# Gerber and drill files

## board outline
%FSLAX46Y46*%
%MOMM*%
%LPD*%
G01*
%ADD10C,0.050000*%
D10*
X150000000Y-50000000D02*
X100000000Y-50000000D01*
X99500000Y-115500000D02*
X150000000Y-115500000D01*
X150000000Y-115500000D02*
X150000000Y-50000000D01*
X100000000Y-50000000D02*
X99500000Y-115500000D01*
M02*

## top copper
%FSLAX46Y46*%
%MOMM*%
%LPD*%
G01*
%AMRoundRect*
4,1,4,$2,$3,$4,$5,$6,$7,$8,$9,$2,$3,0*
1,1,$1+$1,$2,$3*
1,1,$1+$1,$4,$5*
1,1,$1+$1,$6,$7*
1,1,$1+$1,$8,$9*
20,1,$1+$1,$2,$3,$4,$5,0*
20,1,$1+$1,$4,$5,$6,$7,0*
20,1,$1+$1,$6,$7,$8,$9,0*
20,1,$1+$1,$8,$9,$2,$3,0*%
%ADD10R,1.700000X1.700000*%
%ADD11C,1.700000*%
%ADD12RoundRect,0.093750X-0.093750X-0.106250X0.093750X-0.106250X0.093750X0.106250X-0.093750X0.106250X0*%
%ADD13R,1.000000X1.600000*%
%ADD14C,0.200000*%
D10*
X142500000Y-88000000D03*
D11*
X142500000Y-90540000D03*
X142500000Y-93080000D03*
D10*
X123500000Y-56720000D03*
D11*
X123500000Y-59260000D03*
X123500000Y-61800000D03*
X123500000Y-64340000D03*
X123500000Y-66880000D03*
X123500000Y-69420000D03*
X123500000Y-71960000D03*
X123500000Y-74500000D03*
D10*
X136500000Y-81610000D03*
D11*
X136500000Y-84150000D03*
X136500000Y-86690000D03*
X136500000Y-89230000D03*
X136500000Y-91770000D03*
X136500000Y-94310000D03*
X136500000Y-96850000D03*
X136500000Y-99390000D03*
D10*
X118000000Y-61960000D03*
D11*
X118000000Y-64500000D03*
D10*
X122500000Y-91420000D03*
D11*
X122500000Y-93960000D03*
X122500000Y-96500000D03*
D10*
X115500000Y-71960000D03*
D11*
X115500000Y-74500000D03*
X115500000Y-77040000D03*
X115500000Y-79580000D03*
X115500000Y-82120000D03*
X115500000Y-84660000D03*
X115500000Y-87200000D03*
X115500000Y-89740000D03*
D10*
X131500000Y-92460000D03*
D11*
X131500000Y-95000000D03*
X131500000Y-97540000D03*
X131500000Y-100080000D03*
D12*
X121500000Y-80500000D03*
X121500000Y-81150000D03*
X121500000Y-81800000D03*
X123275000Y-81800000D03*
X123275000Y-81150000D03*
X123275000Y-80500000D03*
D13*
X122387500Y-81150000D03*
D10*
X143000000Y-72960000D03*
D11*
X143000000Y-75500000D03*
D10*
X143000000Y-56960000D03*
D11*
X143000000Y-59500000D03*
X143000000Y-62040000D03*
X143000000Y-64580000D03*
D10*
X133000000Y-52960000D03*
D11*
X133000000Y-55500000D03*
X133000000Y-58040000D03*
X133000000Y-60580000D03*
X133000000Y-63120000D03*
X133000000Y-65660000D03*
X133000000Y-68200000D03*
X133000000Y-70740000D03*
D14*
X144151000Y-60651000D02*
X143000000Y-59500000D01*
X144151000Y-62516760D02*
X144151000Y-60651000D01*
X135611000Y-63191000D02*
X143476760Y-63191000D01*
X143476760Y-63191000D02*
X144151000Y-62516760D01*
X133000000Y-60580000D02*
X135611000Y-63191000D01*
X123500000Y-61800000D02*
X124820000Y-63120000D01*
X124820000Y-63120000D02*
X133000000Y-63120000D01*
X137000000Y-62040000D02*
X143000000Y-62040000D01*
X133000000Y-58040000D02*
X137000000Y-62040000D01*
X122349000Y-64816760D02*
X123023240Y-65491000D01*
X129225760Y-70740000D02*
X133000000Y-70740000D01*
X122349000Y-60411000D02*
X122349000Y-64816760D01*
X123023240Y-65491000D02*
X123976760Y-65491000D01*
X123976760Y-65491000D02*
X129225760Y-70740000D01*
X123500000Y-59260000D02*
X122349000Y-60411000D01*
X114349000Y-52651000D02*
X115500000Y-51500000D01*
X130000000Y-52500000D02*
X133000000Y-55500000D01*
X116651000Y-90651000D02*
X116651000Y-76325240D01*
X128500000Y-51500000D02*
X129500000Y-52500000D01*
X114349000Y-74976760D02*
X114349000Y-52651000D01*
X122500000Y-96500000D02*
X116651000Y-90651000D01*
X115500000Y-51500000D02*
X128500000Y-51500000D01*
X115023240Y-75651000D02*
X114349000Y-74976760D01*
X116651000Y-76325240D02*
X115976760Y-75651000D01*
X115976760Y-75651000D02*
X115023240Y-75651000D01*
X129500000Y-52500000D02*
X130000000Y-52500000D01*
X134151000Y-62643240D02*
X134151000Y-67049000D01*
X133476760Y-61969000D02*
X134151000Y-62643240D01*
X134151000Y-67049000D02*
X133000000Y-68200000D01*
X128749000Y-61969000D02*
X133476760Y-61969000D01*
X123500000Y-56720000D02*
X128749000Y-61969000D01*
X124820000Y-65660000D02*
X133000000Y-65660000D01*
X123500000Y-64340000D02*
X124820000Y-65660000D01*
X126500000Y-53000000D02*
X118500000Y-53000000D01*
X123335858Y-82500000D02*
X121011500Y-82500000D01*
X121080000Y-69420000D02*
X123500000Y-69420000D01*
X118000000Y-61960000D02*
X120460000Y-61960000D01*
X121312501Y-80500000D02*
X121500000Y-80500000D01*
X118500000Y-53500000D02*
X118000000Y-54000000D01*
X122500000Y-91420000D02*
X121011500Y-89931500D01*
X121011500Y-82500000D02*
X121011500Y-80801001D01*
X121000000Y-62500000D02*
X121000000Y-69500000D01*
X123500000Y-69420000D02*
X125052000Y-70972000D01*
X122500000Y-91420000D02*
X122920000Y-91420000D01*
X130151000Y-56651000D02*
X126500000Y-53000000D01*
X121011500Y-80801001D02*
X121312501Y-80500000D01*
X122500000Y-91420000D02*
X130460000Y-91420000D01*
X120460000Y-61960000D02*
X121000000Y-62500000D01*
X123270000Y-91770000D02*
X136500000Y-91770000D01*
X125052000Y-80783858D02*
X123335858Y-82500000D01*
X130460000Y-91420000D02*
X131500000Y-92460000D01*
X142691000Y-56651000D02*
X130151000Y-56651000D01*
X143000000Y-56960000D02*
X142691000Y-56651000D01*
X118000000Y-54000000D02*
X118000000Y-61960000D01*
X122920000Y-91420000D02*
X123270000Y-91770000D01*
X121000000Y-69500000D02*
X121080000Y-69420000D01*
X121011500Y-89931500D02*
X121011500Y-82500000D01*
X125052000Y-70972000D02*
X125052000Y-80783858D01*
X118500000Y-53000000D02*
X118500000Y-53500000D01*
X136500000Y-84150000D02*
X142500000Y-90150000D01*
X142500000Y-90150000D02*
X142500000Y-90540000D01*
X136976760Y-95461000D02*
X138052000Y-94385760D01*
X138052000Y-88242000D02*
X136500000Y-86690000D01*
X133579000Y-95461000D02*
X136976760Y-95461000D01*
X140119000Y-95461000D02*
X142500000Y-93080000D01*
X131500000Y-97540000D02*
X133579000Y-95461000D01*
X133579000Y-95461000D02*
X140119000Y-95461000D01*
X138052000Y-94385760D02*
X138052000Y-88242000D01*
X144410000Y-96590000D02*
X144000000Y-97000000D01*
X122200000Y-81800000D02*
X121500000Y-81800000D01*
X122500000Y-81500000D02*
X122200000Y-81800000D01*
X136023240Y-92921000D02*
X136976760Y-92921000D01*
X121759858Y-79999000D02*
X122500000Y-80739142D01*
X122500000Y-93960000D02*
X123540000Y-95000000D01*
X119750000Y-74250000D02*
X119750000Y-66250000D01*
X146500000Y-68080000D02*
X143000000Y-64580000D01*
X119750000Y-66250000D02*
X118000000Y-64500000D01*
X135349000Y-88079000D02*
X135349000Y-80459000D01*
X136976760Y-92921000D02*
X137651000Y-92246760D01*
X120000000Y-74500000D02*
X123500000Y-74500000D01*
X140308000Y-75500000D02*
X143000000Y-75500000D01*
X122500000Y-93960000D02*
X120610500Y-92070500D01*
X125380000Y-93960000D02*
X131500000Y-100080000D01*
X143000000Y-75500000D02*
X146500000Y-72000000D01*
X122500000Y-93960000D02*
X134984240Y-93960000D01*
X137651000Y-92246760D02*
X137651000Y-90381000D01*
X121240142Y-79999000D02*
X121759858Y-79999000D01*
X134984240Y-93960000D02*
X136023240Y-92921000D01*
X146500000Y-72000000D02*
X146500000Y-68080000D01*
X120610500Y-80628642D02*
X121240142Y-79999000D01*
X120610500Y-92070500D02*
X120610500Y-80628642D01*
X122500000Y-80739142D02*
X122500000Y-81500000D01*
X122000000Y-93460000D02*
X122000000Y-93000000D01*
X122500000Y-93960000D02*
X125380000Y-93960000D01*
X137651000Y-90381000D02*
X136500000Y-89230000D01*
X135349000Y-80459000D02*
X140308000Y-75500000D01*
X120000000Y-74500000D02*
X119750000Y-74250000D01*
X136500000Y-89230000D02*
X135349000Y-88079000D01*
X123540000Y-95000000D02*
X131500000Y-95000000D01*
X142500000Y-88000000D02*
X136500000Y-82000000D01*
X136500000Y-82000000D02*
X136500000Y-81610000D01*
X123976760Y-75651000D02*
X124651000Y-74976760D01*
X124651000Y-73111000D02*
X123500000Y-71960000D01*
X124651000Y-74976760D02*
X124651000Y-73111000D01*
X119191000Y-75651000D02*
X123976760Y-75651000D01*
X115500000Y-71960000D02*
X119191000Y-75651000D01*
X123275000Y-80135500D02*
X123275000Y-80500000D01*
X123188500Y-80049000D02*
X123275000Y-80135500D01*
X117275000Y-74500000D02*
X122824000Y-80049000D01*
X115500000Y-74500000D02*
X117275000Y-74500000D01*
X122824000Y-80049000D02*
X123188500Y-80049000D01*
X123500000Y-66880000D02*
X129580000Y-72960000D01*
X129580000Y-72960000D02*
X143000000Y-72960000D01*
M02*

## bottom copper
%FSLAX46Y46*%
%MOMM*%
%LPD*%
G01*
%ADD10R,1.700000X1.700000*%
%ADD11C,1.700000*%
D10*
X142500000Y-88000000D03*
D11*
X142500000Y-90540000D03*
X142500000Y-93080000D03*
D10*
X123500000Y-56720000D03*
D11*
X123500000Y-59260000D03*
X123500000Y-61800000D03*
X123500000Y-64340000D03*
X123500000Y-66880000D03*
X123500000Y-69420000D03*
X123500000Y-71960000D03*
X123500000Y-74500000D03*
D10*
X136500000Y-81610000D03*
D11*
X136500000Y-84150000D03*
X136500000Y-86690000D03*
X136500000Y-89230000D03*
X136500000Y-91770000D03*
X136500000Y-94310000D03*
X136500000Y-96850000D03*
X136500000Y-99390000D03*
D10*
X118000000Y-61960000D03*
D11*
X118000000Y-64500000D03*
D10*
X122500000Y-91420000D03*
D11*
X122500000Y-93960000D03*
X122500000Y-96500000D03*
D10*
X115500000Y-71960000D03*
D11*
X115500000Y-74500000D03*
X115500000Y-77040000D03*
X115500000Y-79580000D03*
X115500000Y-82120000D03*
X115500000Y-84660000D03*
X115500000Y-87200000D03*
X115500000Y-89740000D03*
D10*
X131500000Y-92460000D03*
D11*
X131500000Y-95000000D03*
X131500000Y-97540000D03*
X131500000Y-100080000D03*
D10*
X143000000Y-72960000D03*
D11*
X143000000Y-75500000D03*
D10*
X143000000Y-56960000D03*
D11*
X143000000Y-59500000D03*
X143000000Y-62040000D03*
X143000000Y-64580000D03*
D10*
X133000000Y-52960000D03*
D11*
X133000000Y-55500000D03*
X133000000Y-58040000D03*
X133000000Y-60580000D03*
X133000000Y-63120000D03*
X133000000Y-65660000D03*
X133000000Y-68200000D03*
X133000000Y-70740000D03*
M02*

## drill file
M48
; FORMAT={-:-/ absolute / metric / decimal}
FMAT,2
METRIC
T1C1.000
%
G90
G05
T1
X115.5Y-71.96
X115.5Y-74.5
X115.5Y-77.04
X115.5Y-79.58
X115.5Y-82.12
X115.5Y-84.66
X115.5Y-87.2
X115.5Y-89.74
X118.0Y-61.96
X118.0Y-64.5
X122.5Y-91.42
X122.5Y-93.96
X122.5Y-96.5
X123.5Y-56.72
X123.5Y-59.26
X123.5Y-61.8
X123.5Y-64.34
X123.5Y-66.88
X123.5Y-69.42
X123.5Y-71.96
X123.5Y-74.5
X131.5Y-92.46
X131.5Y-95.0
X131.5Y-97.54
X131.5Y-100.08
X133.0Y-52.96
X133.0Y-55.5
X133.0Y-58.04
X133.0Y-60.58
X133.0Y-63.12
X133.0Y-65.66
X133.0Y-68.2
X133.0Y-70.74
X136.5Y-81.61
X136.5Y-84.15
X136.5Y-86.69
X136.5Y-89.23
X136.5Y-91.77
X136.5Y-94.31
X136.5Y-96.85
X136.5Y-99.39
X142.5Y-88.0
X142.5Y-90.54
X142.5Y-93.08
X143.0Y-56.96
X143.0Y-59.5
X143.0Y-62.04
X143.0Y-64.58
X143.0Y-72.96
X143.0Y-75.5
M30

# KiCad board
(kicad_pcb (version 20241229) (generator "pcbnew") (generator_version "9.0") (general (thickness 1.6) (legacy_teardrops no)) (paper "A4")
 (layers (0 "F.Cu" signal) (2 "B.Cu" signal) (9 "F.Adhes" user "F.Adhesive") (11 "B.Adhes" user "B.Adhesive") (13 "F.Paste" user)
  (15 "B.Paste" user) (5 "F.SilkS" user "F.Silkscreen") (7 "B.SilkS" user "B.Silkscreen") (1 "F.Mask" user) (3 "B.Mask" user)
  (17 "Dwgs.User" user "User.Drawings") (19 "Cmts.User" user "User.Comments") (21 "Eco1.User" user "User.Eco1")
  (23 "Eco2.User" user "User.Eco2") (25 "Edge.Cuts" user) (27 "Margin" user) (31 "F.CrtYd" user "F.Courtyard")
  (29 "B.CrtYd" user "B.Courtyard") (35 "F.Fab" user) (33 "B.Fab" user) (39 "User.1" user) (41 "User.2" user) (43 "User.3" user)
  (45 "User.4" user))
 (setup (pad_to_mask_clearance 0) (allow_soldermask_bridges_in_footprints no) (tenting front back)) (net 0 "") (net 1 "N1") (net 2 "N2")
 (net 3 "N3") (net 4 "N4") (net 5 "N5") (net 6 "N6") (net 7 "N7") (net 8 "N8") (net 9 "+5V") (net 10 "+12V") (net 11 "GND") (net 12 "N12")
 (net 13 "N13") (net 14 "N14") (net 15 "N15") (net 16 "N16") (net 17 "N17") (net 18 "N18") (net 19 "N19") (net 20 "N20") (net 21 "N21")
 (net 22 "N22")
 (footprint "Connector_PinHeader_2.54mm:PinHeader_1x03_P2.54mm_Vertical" (layer "F.Cu") (at 142.5 88)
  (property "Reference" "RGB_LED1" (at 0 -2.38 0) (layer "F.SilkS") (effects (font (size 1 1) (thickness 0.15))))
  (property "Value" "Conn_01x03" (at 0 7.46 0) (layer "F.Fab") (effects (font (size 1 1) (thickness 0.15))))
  (pad "1" thru_hole rect (at 0 0) (size 1.7 1.7) (drill 1) (layers "*.Cu" "*.Mask") (remove_unused_layers no) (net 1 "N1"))
  (pad "2" thru_hole circle (at 0 2.54) (size 1.7 1.7) (drill 1) (layers "*.Cu" "*.Mask") (remove_unused_layers no) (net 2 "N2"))
  (pad "3" thru_hole circle (at 0 5.08) (size 1.7 1.7) (drill 1) (layers "*.Cu" "*.Mask") (remove_unused_layers no) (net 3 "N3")))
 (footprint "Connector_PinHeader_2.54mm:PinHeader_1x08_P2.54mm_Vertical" (layer "F.Cu") (at 123.5 56.72)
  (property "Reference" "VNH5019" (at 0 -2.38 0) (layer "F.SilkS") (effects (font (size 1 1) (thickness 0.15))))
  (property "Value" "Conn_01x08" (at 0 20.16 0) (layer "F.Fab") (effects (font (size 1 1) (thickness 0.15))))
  (pad "1" thru_hole rect (at 0 0) (size 1.7 1.7) (drill 1) (layers "*.Cu" "*.Mask") (remove_unused_layers no) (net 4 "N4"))
  (pad "2" thru_hole circle (at 0 2.54) (size 1.7 1.7) (drill 1) (layers "*.Cu" "*.Mask") (remove_unused_layers no) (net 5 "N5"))
  (pad "3" thru_hole circle (at 0 5.08) (size 1.7 1.7) (drill 1) (layers "*.Cu" "*.Mask") (remove_unused_layers no) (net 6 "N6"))
  (pad "4" thru_hole circle (at 0 7.62) (size 1.7 1.7) (drill 1) (layers "*.Cu" "*.Mask") (remove_unused_layers no) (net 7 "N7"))
  (pad "5" thru_hole circle (at 0 10.16) (size 1.7 1.7) (drill 1) (layers "*.Cu" "*.Mask") (remove_unused_layers no) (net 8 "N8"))
  (pad "6" thru_hole circle (at 0 12.7) (size 1.7 1.7) (drill 1) (layers "*.Cu" "*.Mask") (remove_unused_layers no) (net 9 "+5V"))
  (pad "7" thru_hole circle (at 0 15.24) (size 1.7 1.7) (drill 1) (layers "*.Cu" "*.Mask") (remove_unused_layers no) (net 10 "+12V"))
  (pad "8" thru_hole circle (at 0 17.78) (size 1.7 1.7) (drill 1) (layers "*.Cu" "*.Mask") (remove_unused_layers no) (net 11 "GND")))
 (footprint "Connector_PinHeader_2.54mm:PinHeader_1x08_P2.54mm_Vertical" (layer "F.Cu") (at 136.5 81.61)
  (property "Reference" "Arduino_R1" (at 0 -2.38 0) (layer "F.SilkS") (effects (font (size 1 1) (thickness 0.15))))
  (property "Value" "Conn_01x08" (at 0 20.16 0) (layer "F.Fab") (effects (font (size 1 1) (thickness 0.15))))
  (pad "1" thru_hole rect (at 0 0) (size 1.7 1.7) (drill 1) (layers "*.Cu" "*.Mask") (remove_unused_layers no) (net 1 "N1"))
  (pad "2" thru_hole circle (at 0 2.54) (size 1.7 1.7) (drill 1) (layers "*.Cu" "*.Mask") (remove_unused_layers no) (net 2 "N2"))
  (pad "3" thru_hole circle (at 0 5.08) (size 1.7 1.7) (drill 1) (layers "*.Cu" "*.Mask") (remove_unused_layers no) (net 3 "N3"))
  (pad "4" thru_hole circle (at 0 7.62) (size 1.7 1.7) (drill 1) (layers "*.Cu" "*.Mask") (remove_unused_layers no) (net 11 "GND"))
  (pad "5" thru_hole circle (at 0 10.16) (size 1.7 1.7) (drill 1) (layers "*.Cu" "*.Mask") (remove_unused_layers no) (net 9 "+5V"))
  (pad "6" thru_hole circle (at 0 12.7) (size 1.7 1.7) (drill 1) (layers "*.Cu" "*.Mask") (remove_unused_layers no) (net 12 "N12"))
  (pad "7" thru_hole circle (at 0 15.24) (size 1.7 1.7) (drill 1) (layers "*.Cu" "*.Mask") (remove_unused_layers no) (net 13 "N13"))
  (pad "8" thru_hole circle (at 0 17.78) (size 1.7 1.7) (drill 1) (layers "*.Cu" "*.Mask") (remove_unused_layers no) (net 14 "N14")))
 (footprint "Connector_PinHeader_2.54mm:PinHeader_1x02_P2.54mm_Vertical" (layer "F.Cu") (at 118 61.96)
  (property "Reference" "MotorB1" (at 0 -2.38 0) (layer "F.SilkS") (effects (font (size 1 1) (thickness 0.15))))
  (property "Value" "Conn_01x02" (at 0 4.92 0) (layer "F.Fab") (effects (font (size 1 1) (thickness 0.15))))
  (pad "1" thru_hole rect (at 0 0) (size 1.7 1.7) (drill 1) (layers "*.Cu" "*.Mask") (remove_unused_layers no) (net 9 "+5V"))
  (pad "2" thru_hole circle (at 0 2.54) (size 1.7 1.7) (drill 1) (layers "*.Cu" "*.Mask") (remove_unused_layers no) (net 11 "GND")))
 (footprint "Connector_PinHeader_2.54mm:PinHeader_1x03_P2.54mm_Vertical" (layer "F.Cu") (at 122.5 91.42)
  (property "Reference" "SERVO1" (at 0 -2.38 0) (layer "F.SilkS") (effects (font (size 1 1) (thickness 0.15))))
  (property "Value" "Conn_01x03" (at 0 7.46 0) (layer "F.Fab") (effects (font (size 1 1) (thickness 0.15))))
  (pad "1" thru_hole rect (at 0 0) (size 1.7 1.7) (drill 1) (layers "*.Cu" "*.Mask") (remove_unused_layers no) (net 9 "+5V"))
  (pad "2" thru_hole circle (at 0 2.54) (size 1.7 1.7) (drill 1) (layers "*.Cu" "*.Mask") (remove_unused_layers no) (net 11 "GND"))
  (pad "3" thru_hole circle (at 0 5.08) (size 1.7 1.7) (drill 1) (layers "*.Cu" "*.Mask") (remove_unused_layers no) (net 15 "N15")))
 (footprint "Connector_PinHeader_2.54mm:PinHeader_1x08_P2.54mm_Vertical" (layer "F.Cu") (at 115.5 71.96)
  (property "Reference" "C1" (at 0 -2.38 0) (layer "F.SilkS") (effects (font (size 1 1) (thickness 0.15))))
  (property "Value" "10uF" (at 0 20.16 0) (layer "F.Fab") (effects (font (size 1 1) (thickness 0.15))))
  (pad "1" thru_hole rect (at 0 0) (size 1.7 1.7) (drill 1) (layers "*.Cu" "*.Mask") (remove_unused_layers no) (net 10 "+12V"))
  (pad "2" thru_hole circle (at 0 2.54) (size 1.7 1.7) (drill 1) (layers "*.Cu" "*.Mask") (remove_unused_layers no) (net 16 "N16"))
  (pad "3" thru_hole circle (at 0 5.08) (size 1.7 1.7) (drill 1) (layers "*.Cu" "*.Mask") (remove_unused_layers no))
  (pad "4" thru_hole circle (at 0 7.62) (size 1.7 1.7) (drill 1) (layers "*.Cu" "*.Mask") (remove_unused_layers no))
  (pad "5" thru_hole circle (at 0 10.16) (size 1.7 1.7) (drill 1) (layers "*.Cu" "*.Mask") (remove_unused_layers no))
  (pad "6" thru_hole circle (at 0 12.7) (size 1.7 1.7) (drill 1) (layers "*.Cu" "*.Mask") (remove_unused_layers no))
  (pad "7" thru_hole circle (at 0 15.24) (size 1.7 1.7) (drill 1) (layers "*.Cu" "*.Mask") (remove_unused_layers no))
  (pad "8" thru_hole circle (at 0 17.78) (size 1.7 1.7) (drill 1) (layers "*.Cu" "*.Mask") (remove_unused_layers no)))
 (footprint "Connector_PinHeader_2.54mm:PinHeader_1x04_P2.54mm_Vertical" (layer "F.Cu") (at 131.5 92.46)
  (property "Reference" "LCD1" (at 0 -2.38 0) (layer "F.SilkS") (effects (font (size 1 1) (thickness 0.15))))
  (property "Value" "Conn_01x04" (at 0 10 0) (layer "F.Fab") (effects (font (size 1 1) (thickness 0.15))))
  (pad "1" thru_hole rect (at 0 0) (size 1.7 1.7) (drill 1) (layers "*.Cu" "*.Mask") (remove_unused_layers no) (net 9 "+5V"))
  (pad "2" thru_hole circle (at 0 2.54) (size 1.7 1.7) (drill 1) (layers "*.Cu" "*.Mask") (remove_unused_layers no) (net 11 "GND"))
  (pad "3" thru_hole circle (at 0 5.08) (size 1.7 1.7) (drill 1) (layers "*.Cu" "*.Mask") (remove_unused_layers no) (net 3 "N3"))
  (pad "4" thru_hole circle (at 0 7.62) (size 1.7 1.7) (drill 1) (layers "*.Cu" "*.Mask") (remove_unused_layers no) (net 11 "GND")))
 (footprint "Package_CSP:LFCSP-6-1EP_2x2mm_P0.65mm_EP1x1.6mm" (layer "F.Cu") (at 122.3875 81.15)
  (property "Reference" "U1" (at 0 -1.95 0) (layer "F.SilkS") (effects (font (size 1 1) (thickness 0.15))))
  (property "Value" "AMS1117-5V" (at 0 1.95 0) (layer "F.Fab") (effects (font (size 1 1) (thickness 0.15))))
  (pad "" smd roundrect (at -0.25 -0.4) (size 0.4 0.64) (layers "F.Paste") (roundrect_rratio 0.25))
  (pad "" smd roundrect (at -0.25 0.4) (size 0.4 0.64) (layers "F.Paste") (roundrect_rratio 0.25))
  (pad "" smd roundrect (at 0.25 -0.4) (size 0.4 0.64) (layers "F.Paste") (roundrect_rratio 0.25))
  (pad "" smd roundrect (at 0.25 0.4) (size 0.4 0.64) (layers "F.Paste") (roundrect_rratio 0.25))
  (pad "1" smd roundrect (at -0.8875 -0.65) (size 0.375 0.4) (layers "F.Cu" "F.Mask" "F.Paste") (roundrect_rratio 0.25) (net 9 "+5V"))
  (pad "2" smd roundrect (at -0.8875 0) (size 0.375 0.4) (layers "F.Cu" "F.Mask" "F.Paste") (roundrect_rratio 0.25) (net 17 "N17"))
  (pad "3" smd roundrect (at -0.8875 0.65) (size 0.375 0.4) (layers "F.Cu" "F.Mask" "F.Paste") (roundrect_rratio 0.25) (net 11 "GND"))
  (pad "4" smd roundrect (at 0.8875 0.65) (size 0.375 0.4) (layers "F.Cu" "F.Mask" "F.Paste") (roundrect_rratio 0.25) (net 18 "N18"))
  (pad "5" smd roundrect (at 0.8875 0) (size 0.375 0.4) (layers "F.Cu" "F.Mask" "F.Paste") (roundrect_rratio 0.25) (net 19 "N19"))
  (pad "6" smd roundrect (at 0.8875 -0.65) (size 0.375 0.4) (layers "F.Cu" "F.Mask" "F.Paste") (roundrect_rratio 0.25) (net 16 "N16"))
  (pad "7" smd rect (at 0 0) (size 1 1.6) (layers "F.Cu" "F.Mask") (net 11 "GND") (zone_connect 2)))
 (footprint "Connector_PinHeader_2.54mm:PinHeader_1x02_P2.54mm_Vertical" (layer "F.Cu") (at 143 72.96)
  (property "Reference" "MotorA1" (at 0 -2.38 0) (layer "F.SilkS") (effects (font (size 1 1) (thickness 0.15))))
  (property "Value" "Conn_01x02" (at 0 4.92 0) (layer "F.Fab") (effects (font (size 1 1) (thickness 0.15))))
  (pad "1" thru_hole rect (at 0 0) (size 1.7 1.7) (drill 1) (layers "*.Cu" "*.Mask") (remove_unused_layers no) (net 8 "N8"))
  (pad "2" thru_hole circle (at 0 2.54) (size 1.7 1.7) (drill 1) (layers "*.Cu" "*.Mask") (remove_unused_layers no) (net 11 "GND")))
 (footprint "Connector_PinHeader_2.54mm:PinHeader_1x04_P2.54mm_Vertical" (layer "F.Cu") (at 143 56.96)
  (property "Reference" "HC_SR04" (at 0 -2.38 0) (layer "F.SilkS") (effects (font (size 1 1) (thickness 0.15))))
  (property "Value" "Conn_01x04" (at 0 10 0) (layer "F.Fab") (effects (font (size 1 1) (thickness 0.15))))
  (pad "1" thru_hole rect (at 0 0) (size 1.7 1.7) (drill 1) (layers "*.Cu" "*.Mask") (remove_unused_layers no) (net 9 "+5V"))
  (pad "2" thru_hole circle (at 0 2.54) (size 1.7 1.7) (drill 1) (layers "*.Cu" "*.Mask") (remove_unused_layers no) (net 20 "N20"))
  (pad "3" thru_hole circle (at 0 5.08) (size 1.7 1.7) (drill 1) (layers "*.Cu" "*.Mask") (remove_unused_layers no) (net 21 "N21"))
  (pad "4" thru_hole circle (at 0 7.62) (size 1.7 1.7) (drill 1) (layers "*.Cu" "*.Mask") (remove_unused_layers no) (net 11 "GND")))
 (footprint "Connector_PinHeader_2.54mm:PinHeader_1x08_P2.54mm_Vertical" (layer "F.Cu") (at 133 52.96)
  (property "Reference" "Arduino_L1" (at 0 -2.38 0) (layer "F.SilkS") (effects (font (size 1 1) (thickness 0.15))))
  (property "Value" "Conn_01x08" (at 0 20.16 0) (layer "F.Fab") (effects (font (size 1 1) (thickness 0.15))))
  (pad "1" thru_hole rect (at 0 0) (size 1.7 1.7) (drill 1) (layers "*.Cu" "*.Mask") (remove_unused_layers no) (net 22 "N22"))
  (pad "2" thru_hole circle (at 0 2.54) (size 1.7 1.7) (drill 1) (layers "*.Cu" "*.Mask") (remove_unused_layers no) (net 15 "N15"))
  (pad "3" thru_hole circle (at 0 5.08) (size 1.7 1.7) (drill 1) (layers "*.Cu" "*.Mask") (remove_unused_layers no) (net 21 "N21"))
  (pad "4" thru_hole circle (at 0 7.62) (size 1.7 1.7) (drill 1) (layers "*.Cu" "*.Mask") (remove_unused_layers no) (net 20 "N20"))
  (pad "5" thru_hole circle (at 0 10.16) (size 1.7 1.7) (drill 1) (layers "*.Cu" "*.Mask") (remove_unused_layers no) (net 6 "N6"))
  (pad "6" thru_hole circle (at 0 12.7) (size 1.7 1.7) (drill 1) (layers "*.Cu" "*.Mask") (remove_unused_layers no) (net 7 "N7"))
  (pad "7" thru_hole circle (at 0 15.24) (size 1.7 1.7) (drill 1) (layers "*.Cu" "*.Mask") (remove_unused_layers no) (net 4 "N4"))
  (pad "8" thru_hole circle (at 0 17.78) (size 1.7 1.7) (drill 1) (layers "*.Cu" "*.Mask") (remove_unused_layers no) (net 5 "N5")))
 (gr_line (start 150 50) (end 100 50) (stroke (width 0.05) (type default)) (layer "Edge.Cuts"))
 (gr_line (start 99.5 115.5) (end 150 115.5) (stroke (width 0.05) (type default)) (layer "Edge.Cuts"))
 (gr_line (start 150 115.5) (end 150 50) (stroke (width 0.05) (type default)) (layer "Edge.Cuts"))
 (gr_line (start 100 50) (end 99.5 115.5) (stroke (width 0.05) (type default)) (layer "Edge.Cuts"))
 (segment (start 144.151 60.651) (end 143 59.5) (width 0.2) (layer "F.Cu") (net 20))
 (segment (start 144.151 62.51676) (end 144.151 60.651) (width 0.2) (layer "F.Cu") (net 20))
 (segment (start 135.611 63.191) (end 143.47676 63.191) (width 0.2) (layer "F.Cu") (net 20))
 (segment (start 143.47676 63.191) (end 144.151 62.51676) (width 0.2) (layer "F.Cu") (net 20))
 (segment (start 133 60.58) (end 135.611 63.191) (width 0.2) (layer "F.Cu") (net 20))
 (segment (start 123.5 61.8) (end 124.82 63.12) (width 0.2) (layer "F.Cu") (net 6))
 (segment (start 124.82 63.12) (end 133 63.12) (width 0.2) (layer "F.Cu") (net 6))
 (segment (start 137 62.04) (end 143 62.04) (width 0.2) (layer "F.Cu") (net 21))
 (segment (start 133 58.04) (end 137 62.04) (width 0.2) (layer "F.Cu") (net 21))
 (segment (start 122.349 64.81676) (end 123.02324 65.491) (width 0.2) (layer "F.Cu") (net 5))
 (segment (start 129.22576 70.74) (end 133 70.74) (width 0.2) (layer "F.Cu") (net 5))
 (segment (start 122.349 60.411) (end 122.349 64.81676) (width 0.2) (layer "F.Cu") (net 5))
 (segment (start 123.02324 65.491) (end 123.97676 65.491) (width 0.2) (layer "F.Cu") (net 5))
 (segment (start 123.97676 65.491) (end 129.22576 70.74) (width 0.2) (layer "F.Cu") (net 5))
 (segment (start 123.5 59.26) (end 122.349 60.411) (width 0.2) (layer "F.Cu") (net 5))
 (segment (start 114.349 52.651) (end 115.5 51.5) (width 0.2) (layer "F.Cu") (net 15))
 (segment (start 130 52.5) (end 133 55.5) (width 0.2) (layer "F.Cu") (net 15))
 (segment (start 116.651 90.651) (end 116.651 76.32524) (width 0.2) (layer "F.Cu") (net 15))
 (segment (start 128.5 51.5) (end 129.5 52.5) (width 0.2) (layer "F.Cu") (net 15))
 (segment (start 114.349 74.97676) (end 114.349 52.651) (width 0.2) (layer "F.Cu") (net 15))
 (segment (start 122.5 96.5) (end 116.651 90.651) (width 0.2) (layer "F.Cu") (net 15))
 (segment (start 115.5 51.5) (end 128.5 51.5) (width 0.2) (layer "F.Cu") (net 15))
 (segment (start 115.02324 75.651) (end 114.349 74.97676) (width 0.2) (layer "F.Cu") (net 15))
 (segment (start 116.651 76.32524) (end 115.97676 75.651) (width 0.2) (layer "F.Cu") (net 15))
 (segment (start 115.97676 75.651) (end 115.02324 75.651) (width 0.2) (layer "F.Cu") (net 15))
 (segment (start 129.5 52.5) (end 130 52.5) (width 0.2) (layer "F.Cu") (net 15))
 (segment (start 134.151 62.64324) (end 134.151 67.049) (width 0.2) (layer "F.Cu") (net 4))
 (segment (start 133.47676 61.969) (end 134.151 62.64324) (width 0.2) (layer "F.Cu") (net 4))
 (segment (start 134.151 67.049) (end 133 68.2) (width 0.2) (layer "F.Cu") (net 4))
 (segment (start 128.749 61.969) (end 133.47676 61.969) (width 0.2) (layer "F.Cu") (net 4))
 (segment (start 123.5 56.72) (end 128.749 61.969) (width 0.2) (layer "F.Cu") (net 4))
 (segment (start 124.82 65.66) (end 133 65.66) (width 0.2) (layer "F.Cu") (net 7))
 (segment (start 123.5 64.34) (end 124.82 65.66) (width 0.2) (layer "F.Cu") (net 7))
 (segment (start 126.5 53) (end 118.5 53) (width 0.2) (layer "F.Cu") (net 9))
 (segment (start 123.335858 82.5) (end 121.0115 82.5) (width 0.2) (layer "F.Cu") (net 9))
 (segment (start 121.08 69.42) (end 123.5 69.42) (width 0.2) (layer "F.Cu") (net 9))
 (segment (start 118 61.96) (end 120.46 61.96) (width 0.2) (layer "F.Cu") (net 9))
 (segment (start 121.312501 80.5) (end 121.5 80.5) (width 0.2) (layer "F.Cu") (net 9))
 (segment (start 118.5 53.5) (end 118 54) (width 0.2) (layer "F.Cu") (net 9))
 (segment (start 122.5 91.42) (end 121.0115 89.9315) (width 0.2) (layer "F.Cu") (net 9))
 (segment (start 121.0115 82.5) (end 121.0115 80.801001) (width 0.2) (layer "F.Cu") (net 9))
 (segment (start 121 62.5) (end 121 69.5) (width 0.2) (layer "F.Cu") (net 9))
 (segment (start 123.5 69.42) (end 125.052 70.972) (width 0.2) (layer "F.Cu") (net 9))
 (segment (start 122.5 91.42) (end 122.92 91.42) (width 0.2) (layer "F.Cu") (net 9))
 (segment (start 130.151 56.651) (end 126.5 53) (width 0.2) (layer "F.Cu") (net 9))
 (segment (start 121.0115 80.801001) (end 121.312501 80.5) (width 0.2) (layer "F.Cu") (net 9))
 (segment (start 122.5 91.42) (end 130.46 91.42) (width 0.2) (layer "F.Cu") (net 9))
 (segment (start 120.46 61.96) (end 121 62.5) (width 0.2) (layer "F.Cu") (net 9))
 (segment (start 123.27 91.77) (end 136.5 91.77) (width 0.2) (layer "F.Cu") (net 9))
 (segment (start 125.052 80.783858) (end 123.335858 82.5) (width 0.2) (layer "F.Cu") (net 9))
 (segment (start 130.46 91.42) (end 131.5 92.46) (width 0.2) (layer "F.Cu") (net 9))
 (segment (start 142.691 56.651) (end 130.151 56.651) (width 0.2) (layer "F.Cu") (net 9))
 (segment (start 143 56.96) (end 142.691 56.651) (width 0.2) (layer "F.Cu") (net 9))
 (segment (start 118 54) (end 118 61.96) (width 0.2) (layer "F.Cu") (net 9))
 (segment (start 122.92 91.42) (end 123.27 91.77) (width 0.2) (layer "F.Cu") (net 9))
 (segment (start 121 69.5) (end 121.08 69.42) (width 0.2) (layer "F.Cu") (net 9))
 (segment (start 121.0115 89.9315) (end 121.0115 82.5) (width 0.2) (layer "F.Cu") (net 9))
 (segment (start 125.052 70.972) (end 125.052 80.783858) (width 0.2) (layer "F.Cu") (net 9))
 (segment (start 118.5 53) (end 118.5 53.5) (width 0.2) (layer "F.Cu") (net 9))
 (segment (start 136.5 84.15) (end 142.5 90.15) (width 0.2) (layer "F.Cu") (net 2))
 (segment (start 142.5 90.15) (end 142.5 90.54) (width 0.2) (layer "F.Cu") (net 2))
 (segment (start 136.97676 95.461) (end 138.052 94.38576) (width 0.2) (layer "F.Cu") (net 3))
 (segment (start 138.052 88.242) (end 136.5 86.69) (width 0.2) (layer "F.Cu") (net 3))
 (segment (start 133.579 95.461) (end 136.97676 95.461) (width 0.2) (layer "F.Cu") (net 3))
 (segment (start 140.119 95.461) (end 142.5 93.08) (width 0.2) (layer "F.Cu") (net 3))
 (segment (start 131.5 97.54) (end 133.579 95.461) (width 0.2) (layer "F.Cu") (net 3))
 (segment (start 133.579 95.461) (end 140.119 95.461) (width 0.2) (layer "F.Cu") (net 3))
 (segment (start 138.052 94.38576) (end 138.052 88.242) (width 0.2) (layer "F.Cu") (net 3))
 (segment (start 144.41 96.59) (end 144 97) (width 0.2) (layer "F.Cu") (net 11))
 (segment (start 122.2 81.8) (end 121.5 81.8) (width 0.2) (layer "F.Cu") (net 11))
 (segment (start 122.5 81.5) (end 122.2 81.8) (width 0.2) (layer "F.Cu") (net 11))
 (segment (start 136.02324 92.921) (end 136.97676 92.921) (width 0.2) (layer "F.Cu") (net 11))
 (segment (start 121.759858 79.999) (end 122.5 80.739142) (width 0.2) (layer "F.Cu") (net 11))
 (segment (start 122.5 93.96) (end 123.54 95) (width 0.2) (layer "F.Cu") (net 11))
 (segment (start 119.75 74.25) (end 119.75 66.25) (width 0.2) (layer "F.Cu") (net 11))
 (segment (start 146.5 68.08) (end 143 64.58) (width 0.2) (layer "F.Cu") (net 11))
 (segment (start 119.75 66.25) (end 118 64.5) (width 0.2) (layer "F.Cu") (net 11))
 (segment (start 135.349 88.079) (end 135.349 80.459) (width 0.2) (layer "F.Cu") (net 11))
 (segment (start 136.97676 92.921) (end 137.651 92.24676) (width 0.2) (layer "F.Cu") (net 11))
 (segment (start 120 74.5) (end 123.5 74.5) (width 0.2) (layer "F.Cu") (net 11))
 (segment (start 140.308 75.5) (end 143 75.5) (width 0.2) (layer "F.Cu") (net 11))
 (segment (start 122.5 93.96) (end 120.6105 92.0705) (width 0.2) (layer "F.Cu") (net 11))
 (segment (start 125.38 93.96) (end 131.5 100.08) (width 0.2) (layer "F.Cu") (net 11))
 (segment (start 143 75.5) (end 146.5 72) (width 0.2) (layer "F.Cu") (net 11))
 (segment (start 122.5 93.96) (end 134.98424 93.96) (width 0.2) (layer "F.Cu") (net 11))
 (segment (start 137.651 92.24676) (end 137.651 90.381) (width 0.2) (layer "F.Cu") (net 11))
 (segment (start 121.240142 79.999) (end 121.759858 79.999) (width 0.2) (layer "F.Cu") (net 11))
 (segment (start 134.98424 93.96) (end 136.02324 92.921) (width 0.2) (layer "F.Cu") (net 11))
 (segment (start 146.5 72) (end 146.5 68.08) (width 0.2) (layer "F.Cu") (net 11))
 (segment (start 120.6105 80.628642) (end 121.240142 79.999) (width 0.2) (layer "F.Cu") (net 11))
 (segment (start 120.6105 92.0705) (end 120.6105 80.628642) (width 0.2) (layer "F.Cu") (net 11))
 (segment (start 122.5 80.739142) (end 122.5 81.5) (width 0.2) (layer "F.Cu") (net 11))
 (segment (start 122 93.46) (end 122 93) (width 0.2) (layer "F.Cu") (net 11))
 (segment (start 122.5 93.96) (end 125.38 93.96) (width 0.2) (layer "F.Cu") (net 11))
 (segment (start 137.651 90.381) (end 136.5 89.23) (width 0.2) (layer "F.Cu") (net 11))
 (segment (start 135.349 80.459) (end 140.308 75.5) (width 0.2) (layer "F.Cu") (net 11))
 (segment (start 120 74.5) (end 119.75 74.25) (width 0.2) (layer "F.Cu") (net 11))
 (segment (start 136.5 89.23) (end 135.349 88.079) (width 0.2) (layer "F.Cu") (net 11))
 (segment (start 123.54 95) (end 131.5 95) (width 0.2) (layer "F.Cu") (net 11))
 (segment (start 142.5 88) (end 136.5 82) (width 0.2) (layer "F.Cu") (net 1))
 (segment (start 136.5 82) (end 136.5 81.61) (width 0.2) (layer "F.Cu") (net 1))
 (segment (start 123.97676 75.651) (end 124.651 74.97676) (width 0.2) (layer "F.Cu") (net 10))
 (segment (start 124.651 73.111) (end 123.5 71.96) (width 0.2) (layer "F.Cu") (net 10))
 (segment (start 124.651 74.97676) (end 124.651 73.111) (width 0.2) (layer "F.Cu") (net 10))
 (segment (start 119.191 75.651) (end 123.97676 75.651) (width 0.2) (layer "F.Cu") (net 10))
 (segment (start 115.5 71.96) (end 119.191 75.651) (width 0.2) (layer "F.Cu") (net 10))
 (segment (start 123.275 80.1355) (end 123.275 80.5) (width 0.2) (layer "F.Cu") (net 16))
 (segment (start 123.1885 80.049) (end 123.275 80.1355) (width 0.2) (layer "F.Cu") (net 16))
 (segment (start 117.275 74.5) (end 122.824 80.049) (width 0.2) (layer "F.Cu") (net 16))
 (segment (start 115.5 74.5) (end 117.275 74.5) (width 0.2) (layer "F.Cu") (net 16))
 (segment (start 122.824 80.049) (end 123.1885 80.049) (width 0.2) (layer "F.Cu") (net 16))
 (segment (start 123.5 66.88) (end 129.58 72.96) (width 0.2) (layer "F.Cu") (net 8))
 (segment (start 129.58 72.96) (end 143 72.96) (width 0.2) (layer "F.Cu") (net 8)))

